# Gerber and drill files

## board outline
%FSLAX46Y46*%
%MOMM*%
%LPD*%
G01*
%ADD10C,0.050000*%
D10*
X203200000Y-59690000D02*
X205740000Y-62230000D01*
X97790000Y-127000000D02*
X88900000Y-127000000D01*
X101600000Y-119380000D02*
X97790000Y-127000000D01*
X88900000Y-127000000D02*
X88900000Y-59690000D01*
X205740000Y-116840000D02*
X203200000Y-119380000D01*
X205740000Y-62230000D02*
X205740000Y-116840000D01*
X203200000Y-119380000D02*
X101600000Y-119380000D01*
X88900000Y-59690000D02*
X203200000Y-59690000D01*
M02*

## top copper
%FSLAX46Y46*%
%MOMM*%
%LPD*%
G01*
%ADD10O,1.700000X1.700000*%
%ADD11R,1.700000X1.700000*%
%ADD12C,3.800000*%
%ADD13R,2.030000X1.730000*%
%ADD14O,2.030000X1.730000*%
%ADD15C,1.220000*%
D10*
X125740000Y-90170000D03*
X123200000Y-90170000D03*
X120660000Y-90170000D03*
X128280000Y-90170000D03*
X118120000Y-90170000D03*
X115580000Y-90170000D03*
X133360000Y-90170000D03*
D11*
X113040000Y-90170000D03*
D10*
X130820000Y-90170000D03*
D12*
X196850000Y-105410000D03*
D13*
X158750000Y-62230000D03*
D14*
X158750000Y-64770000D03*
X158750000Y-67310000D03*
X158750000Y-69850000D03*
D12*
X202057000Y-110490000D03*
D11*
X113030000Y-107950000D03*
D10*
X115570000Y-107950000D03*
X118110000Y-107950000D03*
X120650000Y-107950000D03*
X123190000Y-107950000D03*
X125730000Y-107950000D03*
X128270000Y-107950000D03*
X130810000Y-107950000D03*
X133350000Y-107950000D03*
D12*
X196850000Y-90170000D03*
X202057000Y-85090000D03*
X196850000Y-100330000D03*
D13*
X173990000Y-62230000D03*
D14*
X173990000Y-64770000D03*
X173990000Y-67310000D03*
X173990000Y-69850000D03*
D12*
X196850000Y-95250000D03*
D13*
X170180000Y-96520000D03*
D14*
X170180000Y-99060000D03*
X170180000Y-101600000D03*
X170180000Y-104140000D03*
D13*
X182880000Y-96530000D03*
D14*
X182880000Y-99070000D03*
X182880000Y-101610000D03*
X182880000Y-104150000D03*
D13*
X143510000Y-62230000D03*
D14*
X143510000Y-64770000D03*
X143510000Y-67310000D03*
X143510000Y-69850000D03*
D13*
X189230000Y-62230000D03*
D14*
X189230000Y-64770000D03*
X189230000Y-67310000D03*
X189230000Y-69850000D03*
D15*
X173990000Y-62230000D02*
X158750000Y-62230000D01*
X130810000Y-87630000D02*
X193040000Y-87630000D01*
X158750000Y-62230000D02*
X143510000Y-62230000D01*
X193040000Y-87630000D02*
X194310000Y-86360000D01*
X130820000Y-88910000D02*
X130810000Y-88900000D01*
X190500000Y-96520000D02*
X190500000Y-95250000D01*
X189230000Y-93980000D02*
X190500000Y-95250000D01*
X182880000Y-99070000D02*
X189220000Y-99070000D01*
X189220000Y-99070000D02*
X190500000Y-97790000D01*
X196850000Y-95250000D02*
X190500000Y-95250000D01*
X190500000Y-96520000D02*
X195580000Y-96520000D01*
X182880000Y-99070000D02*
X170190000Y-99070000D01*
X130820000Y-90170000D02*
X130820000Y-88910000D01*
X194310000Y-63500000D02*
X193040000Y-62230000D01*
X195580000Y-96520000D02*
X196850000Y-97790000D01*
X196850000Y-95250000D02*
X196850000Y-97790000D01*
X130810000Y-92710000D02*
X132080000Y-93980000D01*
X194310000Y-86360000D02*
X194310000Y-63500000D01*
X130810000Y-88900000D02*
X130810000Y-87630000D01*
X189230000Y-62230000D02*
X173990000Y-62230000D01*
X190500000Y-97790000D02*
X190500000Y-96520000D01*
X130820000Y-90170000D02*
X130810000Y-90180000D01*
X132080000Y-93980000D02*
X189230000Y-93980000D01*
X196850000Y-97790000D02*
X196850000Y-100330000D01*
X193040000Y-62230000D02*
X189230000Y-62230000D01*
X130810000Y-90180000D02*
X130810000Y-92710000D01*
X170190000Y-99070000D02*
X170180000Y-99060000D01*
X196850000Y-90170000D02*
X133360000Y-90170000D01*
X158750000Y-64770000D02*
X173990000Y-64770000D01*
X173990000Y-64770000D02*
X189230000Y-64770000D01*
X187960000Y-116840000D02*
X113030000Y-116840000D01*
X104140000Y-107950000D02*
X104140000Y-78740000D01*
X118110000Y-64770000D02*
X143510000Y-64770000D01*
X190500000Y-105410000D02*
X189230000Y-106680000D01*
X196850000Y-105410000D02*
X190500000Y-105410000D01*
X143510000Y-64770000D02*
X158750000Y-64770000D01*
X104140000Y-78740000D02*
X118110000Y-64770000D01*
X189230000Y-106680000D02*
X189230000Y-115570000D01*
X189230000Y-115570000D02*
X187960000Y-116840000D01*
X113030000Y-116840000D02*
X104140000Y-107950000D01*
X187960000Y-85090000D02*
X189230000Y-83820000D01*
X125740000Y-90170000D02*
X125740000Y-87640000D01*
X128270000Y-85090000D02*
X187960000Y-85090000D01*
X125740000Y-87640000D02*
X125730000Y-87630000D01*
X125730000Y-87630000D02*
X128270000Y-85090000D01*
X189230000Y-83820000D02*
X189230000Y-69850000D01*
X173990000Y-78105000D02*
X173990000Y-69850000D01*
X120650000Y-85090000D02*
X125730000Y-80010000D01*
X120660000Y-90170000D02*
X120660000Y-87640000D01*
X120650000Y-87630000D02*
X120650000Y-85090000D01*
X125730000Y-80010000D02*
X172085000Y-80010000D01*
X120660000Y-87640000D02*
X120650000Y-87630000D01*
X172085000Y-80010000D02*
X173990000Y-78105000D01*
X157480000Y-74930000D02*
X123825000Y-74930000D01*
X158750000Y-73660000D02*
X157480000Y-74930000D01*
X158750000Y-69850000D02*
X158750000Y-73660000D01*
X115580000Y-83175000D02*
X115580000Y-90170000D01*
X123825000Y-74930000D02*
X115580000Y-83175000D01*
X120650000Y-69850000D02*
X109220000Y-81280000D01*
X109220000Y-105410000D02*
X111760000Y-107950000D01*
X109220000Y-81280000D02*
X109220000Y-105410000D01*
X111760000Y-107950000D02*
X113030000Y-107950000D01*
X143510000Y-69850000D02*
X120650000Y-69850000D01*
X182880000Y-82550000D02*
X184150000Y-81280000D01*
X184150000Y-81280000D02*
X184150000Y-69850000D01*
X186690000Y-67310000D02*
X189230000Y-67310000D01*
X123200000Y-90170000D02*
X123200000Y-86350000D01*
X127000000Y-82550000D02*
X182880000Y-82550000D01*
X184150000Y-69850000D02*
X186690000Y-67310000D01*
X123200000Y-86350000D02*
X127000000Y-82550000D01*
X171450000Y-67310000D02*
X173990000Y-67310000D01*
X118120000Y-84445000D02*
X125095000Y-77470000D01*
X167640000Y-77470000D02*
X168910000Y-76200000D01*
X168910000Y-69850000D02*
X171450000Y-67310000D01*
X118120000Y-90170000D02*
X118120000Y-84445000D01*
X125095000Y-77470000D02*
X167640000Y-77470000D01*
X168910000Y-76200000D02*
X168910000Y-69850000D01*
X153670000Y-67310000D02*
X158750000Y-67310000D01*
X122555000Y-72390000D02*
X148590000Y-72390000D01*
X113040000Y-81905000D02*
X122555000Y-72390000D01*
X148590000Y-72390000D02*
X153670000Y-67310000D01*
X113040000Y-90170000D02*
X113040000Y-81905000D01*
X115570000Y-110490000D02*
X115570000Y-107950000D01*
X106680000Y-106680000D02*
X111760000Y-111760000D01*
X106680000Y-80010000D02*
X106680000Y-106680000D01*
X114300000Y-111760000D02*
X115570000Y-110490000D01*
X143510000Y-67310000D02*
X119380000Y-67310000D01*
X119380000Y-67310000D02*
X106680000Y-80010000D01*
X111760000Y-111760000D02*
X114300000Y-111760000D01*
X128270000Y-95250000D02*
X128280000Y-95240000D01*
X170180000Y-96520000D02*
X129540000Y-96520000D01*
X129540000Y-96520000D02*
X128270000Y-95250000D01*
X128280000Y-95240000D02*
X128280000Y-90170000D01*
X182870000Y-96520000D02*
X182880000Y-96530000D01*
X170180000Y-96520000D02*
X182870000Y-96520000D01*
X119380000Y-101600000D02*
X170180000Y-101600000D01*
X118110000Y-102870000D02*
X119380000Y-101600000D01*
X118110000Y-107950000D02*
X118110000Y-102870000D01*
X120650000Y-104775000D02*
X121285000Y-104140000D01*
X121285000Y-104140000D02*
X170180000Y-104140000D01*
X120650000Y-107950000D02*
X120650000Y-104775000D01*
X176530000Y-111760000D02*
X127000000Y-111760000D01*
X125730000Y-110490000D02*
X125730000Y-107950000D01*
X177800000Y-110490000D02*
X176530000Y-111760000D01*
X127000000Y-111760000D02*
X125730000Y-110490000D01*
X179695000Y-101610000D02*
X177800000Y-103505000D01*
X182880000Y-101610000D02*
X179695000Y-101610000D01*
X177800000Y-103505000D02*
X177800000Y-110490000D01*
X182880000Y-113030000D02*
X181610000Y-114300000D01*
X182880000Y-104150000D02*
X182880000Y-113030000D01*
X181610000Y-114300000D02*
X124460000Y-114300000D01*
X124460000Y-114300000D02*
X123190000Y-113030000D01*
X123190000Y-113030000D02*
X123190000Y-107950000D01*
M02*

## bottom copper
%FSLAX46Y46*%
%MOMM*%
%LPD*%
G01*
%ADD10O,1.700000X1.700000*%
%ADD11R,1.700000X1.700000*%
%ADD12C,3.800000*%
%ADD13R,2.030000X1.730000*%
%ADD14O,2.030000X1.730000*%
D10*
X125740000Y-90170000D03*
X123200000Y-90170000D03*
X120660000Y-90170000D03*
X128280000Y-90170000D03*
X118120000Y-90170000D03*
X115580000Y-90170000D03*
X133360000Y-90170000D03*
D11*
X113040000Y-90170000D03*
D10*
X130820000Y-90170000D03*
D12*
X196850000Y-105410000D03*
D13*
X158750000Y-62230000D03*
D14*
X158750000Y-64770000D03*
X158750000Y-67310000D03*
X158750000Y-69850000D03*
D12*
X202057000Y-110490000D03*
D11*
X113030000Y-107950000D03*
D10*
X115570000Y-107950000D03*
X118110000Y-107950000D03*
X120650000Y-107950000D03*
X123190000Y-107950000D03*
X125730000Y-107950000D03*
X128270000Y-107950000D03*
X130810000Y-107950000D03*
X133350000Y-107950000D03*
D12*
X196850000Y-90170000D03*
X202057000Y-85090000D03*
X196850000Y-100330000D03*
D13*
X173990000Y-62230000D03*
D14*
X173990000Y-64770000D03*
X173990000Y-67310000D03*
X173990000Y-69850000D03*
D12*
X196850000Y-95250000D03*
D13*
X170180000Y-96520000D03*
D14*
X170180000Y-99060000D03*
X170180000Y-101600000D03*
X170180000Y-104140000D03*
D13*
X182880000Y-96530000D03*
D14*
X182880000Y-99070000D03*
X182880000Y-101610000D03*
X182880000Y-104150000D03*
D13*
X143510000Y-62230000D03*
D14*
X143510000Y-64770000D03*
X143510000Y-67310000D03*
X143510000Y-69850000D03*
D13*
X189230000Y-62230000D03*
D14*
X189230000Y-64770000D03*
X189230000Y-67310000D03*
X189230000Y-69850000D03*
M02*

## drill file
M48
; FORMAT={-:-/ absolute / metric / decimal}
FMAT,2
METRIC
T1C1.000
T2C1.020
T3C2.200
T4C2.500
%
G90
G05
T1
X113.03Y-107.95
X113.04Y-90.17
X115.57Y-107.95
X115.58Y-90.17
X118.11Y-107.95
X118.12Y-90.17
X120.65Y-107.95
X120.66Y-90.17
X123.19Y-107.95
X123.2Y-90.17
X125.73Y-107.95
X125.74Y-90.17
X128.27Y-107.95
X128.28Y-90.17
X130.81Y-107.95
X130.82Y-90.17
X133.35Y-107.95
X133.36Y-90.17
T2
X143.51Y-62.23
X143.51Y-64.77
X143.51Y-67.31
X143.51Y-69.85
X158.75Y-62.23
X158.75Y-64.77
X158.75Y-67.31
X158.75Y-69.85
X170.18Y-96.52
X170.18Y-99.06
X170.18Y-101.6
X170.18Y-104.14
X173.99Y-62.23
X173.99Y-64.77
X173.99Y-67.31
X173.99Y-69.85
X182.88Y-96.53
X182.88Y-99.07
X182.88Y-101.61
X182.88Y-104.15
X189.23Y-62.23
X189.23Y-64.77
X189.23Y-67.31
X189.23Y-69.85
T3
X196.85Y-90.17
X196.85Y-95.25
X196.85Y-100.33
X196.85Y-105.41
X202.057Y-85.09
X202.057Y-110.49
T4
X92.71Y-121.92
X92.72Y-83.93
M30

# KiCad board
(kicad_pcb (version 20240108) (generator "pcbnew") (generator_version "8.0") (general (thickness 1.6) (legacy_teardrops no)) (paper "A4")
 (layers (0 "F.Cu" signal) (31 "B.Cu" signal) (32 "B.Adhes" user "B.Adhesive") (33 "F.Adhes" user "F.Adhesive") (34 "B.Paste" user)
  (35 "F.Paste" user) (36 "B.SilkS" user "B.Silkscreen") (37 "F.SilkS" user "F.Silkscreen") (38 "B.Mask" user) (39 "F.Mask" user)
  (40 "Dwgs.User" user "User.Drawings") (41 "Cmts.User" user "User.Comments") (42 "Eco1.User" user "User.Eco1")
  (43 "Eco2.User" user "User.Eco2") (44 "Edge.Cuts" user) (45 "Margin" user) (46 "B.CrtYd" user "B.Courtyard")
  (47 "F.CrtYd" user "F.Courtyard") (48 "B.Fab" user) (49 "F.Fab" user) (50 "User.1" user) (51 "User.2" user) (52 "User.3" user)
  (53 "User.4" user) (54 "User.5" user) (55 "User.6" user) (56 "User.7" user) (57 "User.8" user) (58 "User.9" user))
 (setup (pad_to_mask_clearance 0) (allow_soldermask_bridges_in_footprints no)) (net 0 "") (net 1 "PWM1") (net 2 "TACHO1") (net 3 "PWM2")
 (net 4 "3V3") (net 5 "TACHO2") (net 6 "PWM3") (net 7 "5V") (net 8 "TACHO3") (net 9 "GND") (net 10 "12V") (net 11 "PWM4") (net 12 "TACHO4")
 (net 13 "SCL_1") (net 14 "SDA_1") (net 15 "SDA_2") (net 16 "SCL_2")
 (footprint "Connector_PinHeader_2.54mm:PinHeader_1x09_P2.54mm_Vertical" (layer "F.Cu") (at 113.04 90.17 90)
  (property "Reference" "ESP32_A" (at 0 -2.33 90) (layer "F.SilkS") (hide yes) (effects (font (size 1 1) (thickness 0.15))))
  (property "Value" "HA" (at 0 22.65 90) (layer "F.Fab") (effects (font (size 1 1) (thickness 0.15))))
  (pad "1" thru_hole oval (at 0 12.7 90) (size 1.7 1.7) (drill 1) (layers "*.Cu" "*.Mask") (remove_unused_layers no) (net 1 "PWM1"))
  (pad "2" thru_hole oval (at 0 10.16 90) (size 1.7 1.7) (drill 1) (layers "*.Cu" "*.Mask") (remove_unused_layers no) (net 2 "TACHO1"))
  (pad "3" thru_hole oval (at 0 7.62 90) (size 1.7 1.7) (drill 1) (layers "*.Cu" "*.Mask") (remove_unused_layers no) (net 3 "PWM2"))
  (pad "3V3" thru_hole oval (at 0 15.24 90) (size 1.7 1.7) (drill 1) (layers "*.Cu" "*.Mask") (remove_unused_layers no) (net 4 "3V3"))
  (pad "4" thru_hole oval (at 0 5.08 90) (size 1.7 1.7) (drill 1) (layers "*.Cu" "*.Mask") (remove_unused_layers no) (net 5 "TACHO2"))
  (pad "5" thru_hole oval (at 0 2.54 90) (size 1.7 1.7) (drill 1) (layers "*.Cu" "*.Mask") (remove_unused_layers no) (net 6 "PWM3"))
  (pad "5V" thru_hole oval (at 0 20.32 90) (size 1.7 1.7) (drill 1) (layers "*.Cu" "*.Mask") (remove_unused_layers no) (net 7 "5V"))
  (pad "6" thru_hole rect (at 0 0 90) (size 1.7 1.7) (drill 1) (layers "*.Cu" "*.Mask") (remove_unused_layers no) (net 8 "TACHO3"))
  (pad "GND" thru_hole oval (at 0 17.78 90) (size 1.7 1.7) (drill 1) (layers "*.Cu" "*.Mask") (remove_unused_layers no) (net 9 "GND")))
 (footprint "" (layer "F.Cu") (at 196.85 105.41)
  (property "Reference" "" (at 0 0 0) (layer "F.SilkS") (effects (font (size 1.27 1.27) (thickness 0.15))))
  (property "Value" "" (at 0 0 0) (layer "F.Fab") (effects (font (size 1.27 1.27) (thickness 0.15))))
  (pad "1" thru_hole circle (at 0 0) (size 3.8 3.8) (drill 2.2) (layers "*.Cu" "*.Mask") (remove_unused_layers no) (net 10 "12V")))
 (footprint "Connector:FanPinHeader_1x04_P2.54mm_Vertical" (layer "F.Cu") (at 158.75 62.23 -90)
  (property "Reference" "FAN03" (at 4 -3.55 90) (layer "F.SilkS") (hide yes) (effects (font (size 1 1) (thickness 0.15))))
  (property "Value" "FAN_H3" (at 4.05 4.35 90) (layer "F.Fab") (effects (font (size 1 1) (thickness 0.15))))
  (pad "1" thru_hole rect (at 0 0) (size 2.03 1.73) (drill 1.02) (layers "*.Cu" "*.Mask") (remove_unused_layers no) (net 9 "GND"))
  (pad "2" thru_hole oval (at 2.54 0) (size 2.03 1.73) (drill 1.02) (layers "*.Cu" "*.Mask") (remove_unused_layers no) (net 10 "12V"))
  (pad "3" thru_hole oval (at 5.08 0) (size 2.03 1.73) (drill 1.02) (layers "*.Cu" "*.Mask") (remove_unused_layers no) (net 8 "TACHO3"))
  (pad "4" thru_hole oval (at 7.62 0) (size 2.03 1.73) (drill 1.02) (layers "*.Cu" "*.Mask") (remove_unused_layers no) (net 6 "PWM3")))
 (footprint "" (layer "F.Cu") (at 202.057 110.49)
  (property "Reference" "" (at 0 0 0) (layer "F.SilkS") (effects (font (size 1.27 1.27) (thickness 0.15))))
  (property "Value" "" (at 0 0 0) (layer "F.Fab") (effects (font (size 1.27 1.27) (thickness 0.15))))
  (pad "MNT" thru_hole circle (at 0 0) (size 3.8 3.8) (drill 2.2) (layers "*.Cu" "*.Mask") (remove_unused_layers no)))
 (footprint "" (layer "F.Cu") (at 92.71 121.92)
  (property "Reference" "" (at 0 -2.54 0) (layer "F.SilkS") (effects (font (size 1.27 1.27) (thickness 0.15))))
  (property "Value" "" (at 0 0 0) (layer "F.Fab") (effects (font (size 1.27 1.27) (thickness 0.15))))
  (pad "" np_thru_hole circle (at 0 0) (size 2.5 2.5) (drill 2.5) (layers "*.Cu" "*.Mask")))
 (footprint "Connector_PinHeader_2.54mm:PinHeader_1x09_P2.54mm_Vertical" (layer "F.Cu") (at 113.03 107.95 90)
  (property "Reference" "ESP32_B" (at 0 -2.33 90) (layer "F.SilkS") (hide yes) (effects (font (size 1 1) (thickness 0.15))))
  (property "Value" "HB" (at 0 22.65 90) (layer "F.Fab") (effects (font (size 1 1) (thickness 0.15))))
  (pad "7" thru_hole rect (at 0 0 90) (size 1.7 1.7) (drill 1) (layers "*.Cu" "*.Mask") (remove_unused_layers no) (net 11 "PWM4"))
  (pad "8" thru_hole oval (at 0 2.54 90) (size 1.7 1.7) (drill 1) (layers "*.Cu" "*.Mask") (remove_unused_layers no) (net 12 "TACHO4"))
  (pad "9" thru_hole oval (at 0 5.08 90) (size 1.7 1.7) (drill 1) (layers "*.Cu" "*.Mask") (remove_unused_layers no) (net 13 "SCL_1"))
  (pad "10" thru_hole oval (at 0 7.62 90) (size 1.7 1.7) (drill 1) (layers "*.Cu" "*.Mask") (remove_unused_layers no) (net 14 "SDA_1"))
  (pad "11" thru_hole oval (at 0 10.16 90) (size 1.7 1.7) (drill 1) (layers "*.Cu" "*.Mask") (remove_unused_layers no) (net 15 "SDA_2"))
  (pad "12" thru_hole oval (at 0 12.7 90) (size 1.7 1.7) (drill 1) (layers "*.Cu" "*.Mask") (remove_unused_layers no) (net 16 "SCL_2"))
  (pad "13" thru_hole oval (at 0 15.24 90) (size 1.7 1.7) (drill 1) (layers "*.Cu" "*.Mask") (remove_unused_layers no))
  (pad "RX" thru_hole oval (at 0 17.78 90) (size 1.7 1.7) (drill 1) (layers "*.Cu" "*.Mask") (remove_unused_layers no))
  (pad "TX" thru_hole oval (at 0 20.32 90) (size 1.7 1.7) (drill 1) (layers "*.Cu" "*.Mask") (remove_unused_layers no)))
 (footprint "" (layer "F.Cu") (at 196.85 90.17)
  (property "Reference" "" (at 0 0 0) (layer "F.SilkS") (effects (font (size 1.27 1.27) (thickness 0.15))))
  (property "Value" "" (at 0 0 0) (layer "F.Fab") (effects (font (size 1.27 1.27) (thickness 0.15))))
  (pad "4" thru_hole circle (at 0 0) (size 3.8 3.8) (drill 2.2) (layers "*.Cu" "*.Mask") (remove_unused_layers no) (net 7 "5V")))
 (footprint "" (layer "F.Cu") (at 202.057 85.09)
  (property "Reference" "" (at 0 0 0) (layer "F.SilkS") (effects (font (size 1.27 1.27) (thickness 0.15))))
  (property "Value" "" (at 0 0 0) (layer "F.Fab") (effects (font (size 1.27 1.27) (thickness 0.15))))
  (pad "MNT" thru_hole circle (at 0 0) (size 3.8 3.8) (drill 2.2) (layers "*.Cu" "*.Mask") (remove_unused_layers no)))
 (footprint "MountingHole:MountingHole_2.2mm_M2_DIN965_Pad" (layer "F.Cu") (at 196.85 100.33)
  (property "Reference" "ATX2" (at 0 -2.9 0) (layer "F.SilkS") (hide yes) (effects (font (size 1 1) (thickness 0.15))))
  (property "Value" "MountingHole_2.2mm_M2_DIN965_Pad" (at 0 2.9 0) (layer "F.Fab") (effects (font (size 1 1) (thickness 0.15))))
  (pad "2" thru_hole circle (at 0 0) (size 3.8 3.8) (drill 2.2) (layers "*.Cu" "*.Mask") (remove_unused_layers no) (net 9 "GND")))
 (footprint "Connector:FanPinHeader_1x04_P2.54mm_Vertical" (layer "F.Cu") (at 173.99 62.23 -90)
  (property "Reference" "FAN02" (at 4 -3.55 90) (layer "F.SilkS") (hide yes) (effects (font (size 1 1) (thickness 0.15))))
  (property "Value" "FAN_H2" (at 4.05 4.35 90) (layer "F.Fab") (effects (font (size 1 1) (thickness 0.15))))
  (pad "1" thru_hole rect (at 0 0) (size 2.03 1.73) (drill 1.02) (layers "*.Cu" "*.Mask") (remove_unused_layers no) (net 9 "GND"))
  (pad "2" thru_hole oval (at 2.54 0) (size 2.03 1.73) (drill 1.02) (layers "*.Cu" "*.Mask") (remove_unused_layers no) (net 10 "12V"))
  (pad "3" thru_hole oval (at 5.08 0) (size 2.03 1.73) (drill 1.02) (layers "*.Cu" "*.Mask") (remove_unused_layers no) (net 5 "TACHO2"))
  (pad "4" thru_hole oval (at 7.62 0) (size 2.03 1.73) (drill 1.02) (layers "*.Cu" "*.Mask") (remove_unused_layers no) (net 3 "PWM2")))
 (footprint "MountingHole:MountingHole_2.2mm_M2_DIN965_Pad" (layer "F.Cu") (at 196.85 95.25)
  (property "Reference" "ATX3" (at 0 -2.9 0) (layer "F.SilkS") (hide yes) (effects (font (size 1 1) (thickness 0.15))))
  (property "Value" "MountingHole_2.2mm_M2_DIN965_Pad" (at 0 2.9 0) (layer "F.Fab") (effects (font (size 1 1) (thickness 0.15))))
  (pad "3" thru_hole circle (at 0 0) (size 3.8 3.8) (drill 2.2) (layers "*.Cu" "*.Mask") (remove_unused_layers no) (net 9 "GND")))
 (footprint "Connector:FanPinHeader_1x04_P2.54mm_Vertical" (layer "F.Cu") (at 170.18 96.52 -90)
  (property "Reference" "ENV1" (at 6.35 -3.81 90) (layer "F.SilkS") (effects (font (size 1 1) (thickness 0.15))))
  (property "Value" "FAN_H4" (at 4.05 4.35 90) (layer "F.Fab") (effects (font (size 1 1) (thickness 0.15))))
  (pad "1" thru_hole rect (at 0 0) (size 2.03 1.73) (drill 1.02) (layers "*.Cu" "*.Mask") (remove_unused_layers no) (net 4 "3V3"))
  (pad "2" thru_hole oval (at 2.54 0) (size 2.03 1.73) (drill 1.02) (layers "*.Cu" "*.Mask") (remove_unused_layers no) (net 9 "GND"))
  (pad "3" thru_hole oval (at 5.08 0) (size 2.03 1.73) (drill 1.02) (layers "*.Cu" "*.Mask") (remove_unused_layers no) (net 13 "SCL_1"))
  (pad "4" thru_hole oval (at 7.62 0) (size 2.03 1.73) (drill 1.02) (layers "*.Cu" "*.Mask") (remove_unused_layers no) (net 14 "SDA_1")))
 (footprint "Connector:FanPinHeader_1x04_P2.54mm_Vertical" (layer "F.Cu") (at 182.88 96.53 -90)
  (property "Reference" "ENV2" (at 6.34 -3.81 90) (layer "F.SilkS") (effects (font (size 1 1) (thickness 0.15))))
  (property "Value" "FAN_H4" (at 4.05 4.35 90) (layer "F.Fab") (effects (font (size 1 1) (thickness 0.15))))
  (pad "1" thru_hole rect (at 0 0) (size 2.03 1.73) (drill 1.02) (layers "*.Cu" "*.Mask") (remove_unused_layers no) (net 4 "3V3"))
  (pad "2" thru_hole oval (at 2.54 0) (size 2.03 1.73) (drill 1.02) (layers "*.Cu" "*.Mask") (remove_unused_layers no) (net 9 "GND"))
  (pad "3" thru_hole oval (at 5.08 0) (size 2.03 1.73) (drill 1.02) (layers "*.Cu" "*.Mask") (remove_unused_layers no) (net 16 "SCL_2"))
  (pad "4" thru_hole oval (at 7.62 0) (size 2.03 1.73) (drill 1.02) (layers "*.Cu" "*.Mask") (remove_unused_layers no) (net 15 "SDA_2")))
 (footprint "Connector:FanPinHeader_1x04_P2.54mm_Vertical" (layer "F.Cu") (at 143.51 62.23 -90)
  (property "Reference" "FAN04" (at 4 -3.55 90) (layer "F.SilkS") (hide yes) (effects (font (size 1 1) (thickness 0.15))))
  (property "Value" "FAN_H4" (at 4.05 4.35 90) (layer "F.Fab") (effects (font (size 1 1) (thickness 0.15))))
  (pad "1" thru_hole rect (at 0 0) (size 2.03 1.73) (drill 1.02) (layers "*.Cu" "*.Mask") (remove_unused_layers no) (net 9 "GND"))
  (pad "2" thru_hole oval (at 2.54 0) (size 2.03 1.73) (drill 1.02) (layers "*.Cu" "*.Mask") (remove_unused_layers no) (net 10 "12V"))
  (pad "3" thru_hole oval (at 5.08 0) (size 2.03 1.73) (drill 1.02) (layers "*.Cu" "*.Mask") (remove_unused_layers no) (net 12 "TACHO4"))
  (pad "4" thru_hole oval (at 7.62 0) (size 2.03 1.73) (drill 1.02) (layers "*.Cu" "*.Mask") (remove_unused_layers no) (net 11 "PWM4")))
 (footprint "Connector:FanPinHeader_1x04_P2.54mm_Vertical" (layer "F.Cu") (at 189.23 62.23 -90)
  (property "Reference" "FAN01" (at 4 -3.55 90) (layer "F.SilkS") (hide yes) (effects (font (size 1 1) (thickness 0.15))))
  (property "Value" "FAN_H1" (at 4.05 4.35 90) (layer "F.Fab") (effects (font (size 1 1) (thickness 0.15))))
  (pad "1" thru_hole rect (at 0 0) (size 2.03 1.73) (drill 1.02) (layers "*.Cu" "*.Mask") (remove_unused_layers no) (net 9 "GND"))
  (pad "2" thru_hole oval (at 2.54 0) (size 2.03 1.73) (drill 1.02) (layers "*.Cu" "*.Mask") (remove_unused_layers no) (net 10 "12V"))
  (pad "3" thru_hole oval (at 5.08 0) (size 2.03 1.73) (drill 1.02) (layers "*.Cu" "*.Mask") (remove_unused_layers no) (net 2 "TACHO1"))
  (pad "4" thru_hole oval (at 7.62 0) (size 2.03 1.73) (drill 1.02) (layers "*.Cu" "*.Mask") (remove_unused_layers no) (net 1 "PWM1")))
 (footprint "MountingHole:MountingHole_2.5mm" (layer "F.Cu") (at 92.72 83.93)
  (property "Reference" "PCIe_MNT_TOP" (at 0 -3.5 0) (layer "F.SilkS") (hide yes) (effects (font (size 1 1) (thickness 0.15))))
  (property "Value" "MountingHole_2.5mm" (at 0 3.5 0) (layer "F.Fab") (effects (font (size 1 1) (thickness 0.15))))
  (pad "" np_thru_hole circle (at 0 0) (size 2.5 2.5) (drill 2.5) (layers "*.Cu" "*.Mask")))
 (gr_line (start 203.2 59.69) (end 205.74 62.23) (stroke (width 0.05) (type default)) (layer "Edge.Cuts"))
 (gr_line (start 97.79 127) (end 88.9 127) (stroke (width 0.05) (type default)) (layer "Edge.Cuts"))
 (gr_line (start 101.6 119.38) (end 97.79 127) (stroke (width 0.05) (type default)) (layer "Edge.Cuts"))
 (gr_line (start 88.9 127) (end 88.9 59.69) (stroke (width 0.05) (type default)) (layer "Edge.Cuts"))
 (gr_line (start 205.74 116.84) (end 203.2 119.38) (stroke (width 0.05) (type default)) (layer "Edge.Cuts"))
 (gr_line (start 205.74 62.23) (end 205.74 116.84) (stroke (width 0.05) (type default)) (layer "Edge.Cuts"))
 (gr_line (start 203.2 119.38) (end 101.6 119.38) (stroke (width 0.05) (type default)) (layer "Edge.Cuts"))
 (gr_line (start 88.9 59.69) (end 203.2 59.69) (stroke (width 0.05) (type default)) (layer "Edge.Cuts"))
 (segment (start 173.99 62.23) (end 158.75 62.23) (width 1.22) (layer "F.Cu") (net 9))
 (segment (start 130.81 87.63) (end 193.04 87.63) (width 1.22) (layer "F.Cu") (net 9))
 (segment (start 158.75 62.23) (end 143.51 62.23) (width 1.22) (layer "F.Cu") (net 9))
 (segment (start 193.04 87.63) (end 194.31 86.36) (width 1.22) (layer "F.Cu") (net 9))
 (segment (start 130.82 88.91) (end 130.81 88.9) (width 1.22) (layer "F.Cu") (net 9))
 (segment (start 190.5 96.52) (end 190.5 95.25) (width 1.22) (layer "F.Cu") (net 9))
 (segment (start 189.23 93.98) (end 190.5 95.25) (width 1.22) (layer "F.Cu") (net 9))
 (segment (start 182.88 99.07) (end 189.22 99.07) (width 1.22) (layer "F.Cu") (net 9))
 (segment (start 189.22 99.07) (end 190.5 97.79) (width 1.22) (layer "F.Cu") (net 9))
 (segment (start 196.85 95.25) (end 190.5 95.25) (width 1.22) (layer "F.Cu") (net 9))
 (segment (start 190.5 96.52) (end 195.58 96.52) (width 1.22) (layer "F.Cu") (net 9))
 (segment (start 182.88 99.07) (end 170.19 99.07) (width 1.22) (layer "F.Cu") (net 9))
 (segment (start 130.82 90.17) (end 130.82 88.91) (width 1.22) (layer "F.Cu") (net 9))
 (segment (start 194.31 63.5) (end 193.04 62.23) (width 1.22) (layer "F.Cu") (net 9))
 (segment (start 195.58 96.52) (end 196.85 97.79) (width 1.22) (layer "F.Cu") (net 9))
 (segment (start 196.85 95.25) (end 196.85 97.79) (width 1.22) (layer "F.Cu") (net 9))
 (segment (start 130.81 92.71) (end 132.08 93.98) (width 1.22) (layer "F.Cu") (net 9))
 (segment (start 194.31 86.36) (end 194.31 63.5) (width 1.22) (layer "F.Cu") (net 9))
 (segment (start 130.81 88.9) (end 130.81 87.63) (width 1.22) (layer "F.Cu") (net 9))
 (segment (start 189.23 62.23) (end 173.99 62.23) (width 1.22) (layer "F.Cu") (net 9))
 (segment (start 190.5 97.79) (end 190.5 96.52) (width 1.22) (layer "F.Cu") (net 9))
 (segment (start 130.82 90.17) (end 130.81 90.18) (width 1.22) (layer "F.Cu") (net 9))
 (segment (start 132.08 93.98) (end 189.23 93.98) (width 1.22) (layer "F.Cu") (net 9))
 (segment (start 196.85 97.79) (end 196.85 100.33) (width 1.22) (layer "F.Cu") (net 9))
 (segment (start 193.04 62.23) (end 189.23 62.23) (width 1.22) (layer "F.Cu") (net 9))
 (segment (start 130.81 90.18) (end 130.81 92.71) (width 1.22) (layer "F.Cu") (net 9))
 (segment (start 170.19 99.07) (end 170.18 99.06) (width 1.22) (layer "F.Cu") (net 9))
 (segment (start 196.85 90.17) (end 133.36 90.17) (width 1.22) (layer "F.Cu") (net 7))
 (segment (start 158.75 64.77) (end 173.99 64.77) (width 1.22) (layer "F.Cu") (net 10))
 (segment (start 173.99 64.77) (end 189.23 64.77) (width 1.22) (layer "F.Cu") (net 10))
 (segment (start 187.96 116.84) (end 113.03 116.84) (width 1.22) (layer "F.Cu") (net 10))
 (segment (start 104.14 107.95) (end 104.14 78.74) (width 1.22) (layer "F.Cu") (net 10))
 (segment (start 118.11 64.77) (end 143.51 64.77) (width 1.22) (layer "F.Cu") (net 10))
 (segment (start 190.5 105.41) (end 189.23 106.68) (width 1.22) (layer "F.Cu") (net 10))
 (segment (start 196.85 105.41) (end 190.5 105.41) (width 1.22) (layer "F.Cu") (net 10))
 (segment (start 143.51 64.77) (end 158.75 64.77) (width 1.22) (layer "F.Cu") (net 10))
 (segment (start 104.14 78.74) (end 118.11 64.77) (width 1.22) (layer "F.Cu") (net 10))
 (segment (start 189.23 106.68) (end 189.23 115.57) (width 1.22) (layer "F.Cu") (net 10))
 (segment (start 189.23 115.57) (end 187.96 116.84) (width 1.22) (layer "F.Cu") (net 10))
 (segment (start 113.03 116.84) (end 104.14 107.95) (width 1.22) (layer "F.Cu") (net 10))
 (segment (start 187.96 85.09) (end 189.23 83.82) (width 1.22) (layer "F.Cu") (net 1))
 (segment (start 125.74 90.17) (end 125.74 87.64) (width 1.22) (layer "F.Cu") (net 1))
 (segment (start 128.27 85.09) (end 187.96 85.09) (width 1.22) (layer "F.Cu") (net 1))
 (segment (start 125.74 87.64) (end 125.73 87.63) (width 1.22) (layer "F.Cu") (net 1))
 (segment (start 125.73 87.63) (end 128.27 85.09) (width 1.22) (layer "F.Cu") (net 1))
 (segment (start 189.23 83.82) (end 189.23 69.85) (width 1.22) (layer "F.Cu") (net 1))
 (segment (start 173.99 78.105) (end 173.99 69.85) (width 1.22) (layer "F.Cu") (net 3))
 (segment (start 120.65 85.09) (end 125.73 80.01) (width 1.22) (layer "F.Cu") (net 3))
 (segment (start 120.66 90.17) (end 120.66 87.64) (width 1.22) (layer "F.Cu") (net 3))
 (segment (start 120.65 87.63) (end 120.65 85.09) (width 1.22) (layer "F.Cu") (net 3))
 (segment (start 125.73 80.01) (end 172.085 80.01) (width 1.22) (layer "F.Cu") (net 3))
 (segment (start 120.66 87.64) (end 120.65 87.63) (width 1.22) (layer "F.Cu") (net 3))
 (segment (start 172.085 80.01) (end 173.99 78.105) (width 1.22) (layer "F.Cu") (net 3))
 (segment (start 157.48 74.93) (end 123.825 74.93) (width 1.22) (layer "F.Cu") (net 6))
 (segment (start 158.75 73.66) (end 157.48 74.93) (width 1.22) (layer "F.Cu") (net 6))
 (segment (start 158.75 69.85) (end 158.75 73.66) (width 1.22) (layer "F.Cu") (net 6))
 (segment (start 115.58 83.175) (end 115.58 90.17) (width 1.22) (layer "F.Cu") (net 6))
 (segment (start 123.825 74.93) (end 115.58 83.175) (width 1.22) (layer "F.Cu") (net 6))
 (segment (start 120.65 69.85) (end 109.22 81.28) (width 1.22) (layer "F.Cu") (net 11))
 (segment (start 109.22 105.41) (end 111.76 107.95) (width 1.22) (layer "F.Cu") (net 11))
 (segment (start 109.22 81.28) (end 109.22 105.41) (width 1.22) (layer "F.Cu") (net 11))
 (segment (start 111.76 107.95) (end 113.03 107.95) (width 1.22) (layer "F.Cu") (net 11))
 (segment (start 143.51 69.85) (end 120.65 69.85) (width 1.22) (layer "F.Cu") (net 11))
 (segment (start 182.88 82.55) (end 184.15 81.28) (width 1.22) (layer "F.Cu") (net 2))
 (segment (start 184.15 81.28) (end 184.15 69.85) (width 1.22) (layer "F.Cu") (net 2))
 (segment (start 186.69 67.31) (end 189.23 67.31) (width 1.22) (layer "F.Cu") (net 2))
 (segment (start 123.2 90.17) (end 123.2 86.35) (width 1.22) (layer "F.Cu") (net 2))
 (segment (start 127 82.55) (end 182.88 82.55) (width 1.22) (layer "F.Cu") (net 2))
 (segment (start 184.15 69.85) (end 186.69 67.31) (width 1.22) (layer "F.Cu") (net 2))
 (segment (start 123.2 86.35) (end 127 82.55) (width 1.22) (layer "F.Cu") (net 2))
 (segment (start 171.45 67.31) (end 173.99 67.31) (width 1.22) (layer "F.Cu") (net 5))
 (segment (start 118.12 84.445) (end 125.095 77.47) (width 1.22) (layer "F.Cu") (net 5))
 (segment (start 167.64 77.47) (end 168.91 76.2) (width 1.22) (layer "F.Cu") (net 5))
 (segment (start 168.91 69.85) (end 171.45 67.31) (width 1.22) (layer "F.Cu") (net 5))
 (segment (start 118.12 90.17) (end 118.12 84.445) (width 1.22) (layer "F.Cu") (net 5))
 (segment (start 125.095 77.47) (end 167.64 77.47) (width 1.22) (layer "F.Cu") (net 5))
 (segment (start 168.91 76.2) (end 168.91 69.85) (width 1.22) (layer "F.Cu") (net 5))
 (segment (start 153.67 67.31) (end 158.75 67.31) (width 1.22) (layer "F.Cu") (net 8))
 (segment (start 122.555 72.39) (end 148.59 72.39) (width 1.22) (layer "F.Cu") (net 8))
 (segment (start 113.04 81.905) (end 122.555 72.39) (width 1.22) (layer "F.Cu") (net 8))
 (segment (start 148.59 72.39) (end 153.67 67.31) (width 1.22) (layer "F.Cu") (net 8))
 (segment (start 113.04 90.17) (end 113.04 81.905) (width 1.22) (layer "F.Cu") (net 8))
 (segment (start 115.57 110.49) (end 115.57 107.95) (width 1.22) (layer "F.Cu") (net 12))
 (segment (start 106.68 106.68) (end 111.76 111.76) (width 1.22) (layer "F.Cu") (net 12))
 (segment (start 106.68 80.01) (end 106.68 106.68) (width 1.22) (layer "F.Cu") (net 12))
 (segment (start 114.3 111.76) (end 115.57 110.49) (width 1.22) (layer "F.Cu") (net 12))
 (segment (start 143.51 67.31) (end 119.38 67.31) (width 1.22) (layer "F.Cu") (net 12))
 (segment (start 119.38 67.31) (end 106.68 80.01) (width 1.22) (layer "F.Cu") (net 12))
 (segment (start 111.76 111.76) (end 114.3 111.76) (width 1.22) (layer "F.Cu") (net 12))
 (segment (start 128.27 95.25) (end 128.28 95.24) (width 1.22) (layer "F.Cu") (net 4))
 (segment (start 170.18 96.52) (end 129.54 96.52) (width 1.22) (layer "F.Cu") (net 4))
 (segment (start 129.54 96.52) (end 128.27 95.25) (width 1.22) (layer "F.Cu") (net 4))
 (segment (start 128.28 95.24) (end 128.28 90.17) (width 1.22) (layer "F.Cu") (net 4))
 (segment (start 182.87 96.52) (end 182.88 96.53) (width 1.22) (layer "F.Cu") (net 4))
 (segment (start 170.18 96.52) (end 182.87 96.52) (width 1.22) (layer "F.Cu") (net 4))
 (segment (start 119.38 101.6) (end 170.18 101.6) (width 1.22) (layer "F.Cu") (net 13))
 (segment (start 118.11 102.87) (end 119.38 101.6) (width 1.22) (layer "F.Cu") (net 13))
 (segment (start 118.11 107.95) (end 118.11 102.87) (width 1.22) (layer "F.Cu") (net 13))
 (segment (start 120.65 104.775) (end 121.285 104.14) (width 1.22) (layer "F.Cu") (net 14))
 (segment (start 121.285 104.14) (end 170.18 104.14) (width 1.22) (layer "F.Cu") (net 14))
 (segment (start 120.65 107.95) (end 120.65 104.775) (width 1.22) (layer "F.Cu") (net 14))
 (segment (start 176.53 111.76) (end 127 111.76) (width 1.22) (layer "F.Cu") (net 16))
 (segment (start 125.73 110.49) (end 125.73 107.95) (width 1.22) (layer "F.Cu") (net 16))
 (segment (start 177.8 110.49) (end 176.53 111.76) (width 1.22) (layer "F.Cu") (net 16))
 (segment (start 127 111.76) (end 125.73 110.49) (width 1.22) (layer "F.Cu") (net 16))
 (segment (start 179.695 101.61) (end 177.8 103.505) (width 1.22) (layer "F.Cu") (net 16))
 (segment (start 182.88 101.61) (end 179.695 101.61) (width 1.22) (layer "F.Cu") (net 16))
 (segment (start 177.8 103.505) (end 177.8 110.49) (width 1.22) (layer "F.Cu") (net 16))
 (segment (start 182.88 113.03) (end 181.61 114.3) (width 1.22) (layer "F.Cu") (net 15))
 (segment (start 182.88 104.15) (end 182.88 113.03) (width 1.22) (layer "F.Cu") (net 15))
 (segment (start 181.61 114.3) (end 124.46 114.3) (width 1.22) (layer "F.Cu") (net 15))
 (segment (start 124.46 114.3) (end 123.19 113.03) (width 1.22) (layer "F.Cu") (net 15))
 (segment (start 123.19 113.03) (end 123.19 107.95) (width 1.22) (layer "F.Cu") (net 15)))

